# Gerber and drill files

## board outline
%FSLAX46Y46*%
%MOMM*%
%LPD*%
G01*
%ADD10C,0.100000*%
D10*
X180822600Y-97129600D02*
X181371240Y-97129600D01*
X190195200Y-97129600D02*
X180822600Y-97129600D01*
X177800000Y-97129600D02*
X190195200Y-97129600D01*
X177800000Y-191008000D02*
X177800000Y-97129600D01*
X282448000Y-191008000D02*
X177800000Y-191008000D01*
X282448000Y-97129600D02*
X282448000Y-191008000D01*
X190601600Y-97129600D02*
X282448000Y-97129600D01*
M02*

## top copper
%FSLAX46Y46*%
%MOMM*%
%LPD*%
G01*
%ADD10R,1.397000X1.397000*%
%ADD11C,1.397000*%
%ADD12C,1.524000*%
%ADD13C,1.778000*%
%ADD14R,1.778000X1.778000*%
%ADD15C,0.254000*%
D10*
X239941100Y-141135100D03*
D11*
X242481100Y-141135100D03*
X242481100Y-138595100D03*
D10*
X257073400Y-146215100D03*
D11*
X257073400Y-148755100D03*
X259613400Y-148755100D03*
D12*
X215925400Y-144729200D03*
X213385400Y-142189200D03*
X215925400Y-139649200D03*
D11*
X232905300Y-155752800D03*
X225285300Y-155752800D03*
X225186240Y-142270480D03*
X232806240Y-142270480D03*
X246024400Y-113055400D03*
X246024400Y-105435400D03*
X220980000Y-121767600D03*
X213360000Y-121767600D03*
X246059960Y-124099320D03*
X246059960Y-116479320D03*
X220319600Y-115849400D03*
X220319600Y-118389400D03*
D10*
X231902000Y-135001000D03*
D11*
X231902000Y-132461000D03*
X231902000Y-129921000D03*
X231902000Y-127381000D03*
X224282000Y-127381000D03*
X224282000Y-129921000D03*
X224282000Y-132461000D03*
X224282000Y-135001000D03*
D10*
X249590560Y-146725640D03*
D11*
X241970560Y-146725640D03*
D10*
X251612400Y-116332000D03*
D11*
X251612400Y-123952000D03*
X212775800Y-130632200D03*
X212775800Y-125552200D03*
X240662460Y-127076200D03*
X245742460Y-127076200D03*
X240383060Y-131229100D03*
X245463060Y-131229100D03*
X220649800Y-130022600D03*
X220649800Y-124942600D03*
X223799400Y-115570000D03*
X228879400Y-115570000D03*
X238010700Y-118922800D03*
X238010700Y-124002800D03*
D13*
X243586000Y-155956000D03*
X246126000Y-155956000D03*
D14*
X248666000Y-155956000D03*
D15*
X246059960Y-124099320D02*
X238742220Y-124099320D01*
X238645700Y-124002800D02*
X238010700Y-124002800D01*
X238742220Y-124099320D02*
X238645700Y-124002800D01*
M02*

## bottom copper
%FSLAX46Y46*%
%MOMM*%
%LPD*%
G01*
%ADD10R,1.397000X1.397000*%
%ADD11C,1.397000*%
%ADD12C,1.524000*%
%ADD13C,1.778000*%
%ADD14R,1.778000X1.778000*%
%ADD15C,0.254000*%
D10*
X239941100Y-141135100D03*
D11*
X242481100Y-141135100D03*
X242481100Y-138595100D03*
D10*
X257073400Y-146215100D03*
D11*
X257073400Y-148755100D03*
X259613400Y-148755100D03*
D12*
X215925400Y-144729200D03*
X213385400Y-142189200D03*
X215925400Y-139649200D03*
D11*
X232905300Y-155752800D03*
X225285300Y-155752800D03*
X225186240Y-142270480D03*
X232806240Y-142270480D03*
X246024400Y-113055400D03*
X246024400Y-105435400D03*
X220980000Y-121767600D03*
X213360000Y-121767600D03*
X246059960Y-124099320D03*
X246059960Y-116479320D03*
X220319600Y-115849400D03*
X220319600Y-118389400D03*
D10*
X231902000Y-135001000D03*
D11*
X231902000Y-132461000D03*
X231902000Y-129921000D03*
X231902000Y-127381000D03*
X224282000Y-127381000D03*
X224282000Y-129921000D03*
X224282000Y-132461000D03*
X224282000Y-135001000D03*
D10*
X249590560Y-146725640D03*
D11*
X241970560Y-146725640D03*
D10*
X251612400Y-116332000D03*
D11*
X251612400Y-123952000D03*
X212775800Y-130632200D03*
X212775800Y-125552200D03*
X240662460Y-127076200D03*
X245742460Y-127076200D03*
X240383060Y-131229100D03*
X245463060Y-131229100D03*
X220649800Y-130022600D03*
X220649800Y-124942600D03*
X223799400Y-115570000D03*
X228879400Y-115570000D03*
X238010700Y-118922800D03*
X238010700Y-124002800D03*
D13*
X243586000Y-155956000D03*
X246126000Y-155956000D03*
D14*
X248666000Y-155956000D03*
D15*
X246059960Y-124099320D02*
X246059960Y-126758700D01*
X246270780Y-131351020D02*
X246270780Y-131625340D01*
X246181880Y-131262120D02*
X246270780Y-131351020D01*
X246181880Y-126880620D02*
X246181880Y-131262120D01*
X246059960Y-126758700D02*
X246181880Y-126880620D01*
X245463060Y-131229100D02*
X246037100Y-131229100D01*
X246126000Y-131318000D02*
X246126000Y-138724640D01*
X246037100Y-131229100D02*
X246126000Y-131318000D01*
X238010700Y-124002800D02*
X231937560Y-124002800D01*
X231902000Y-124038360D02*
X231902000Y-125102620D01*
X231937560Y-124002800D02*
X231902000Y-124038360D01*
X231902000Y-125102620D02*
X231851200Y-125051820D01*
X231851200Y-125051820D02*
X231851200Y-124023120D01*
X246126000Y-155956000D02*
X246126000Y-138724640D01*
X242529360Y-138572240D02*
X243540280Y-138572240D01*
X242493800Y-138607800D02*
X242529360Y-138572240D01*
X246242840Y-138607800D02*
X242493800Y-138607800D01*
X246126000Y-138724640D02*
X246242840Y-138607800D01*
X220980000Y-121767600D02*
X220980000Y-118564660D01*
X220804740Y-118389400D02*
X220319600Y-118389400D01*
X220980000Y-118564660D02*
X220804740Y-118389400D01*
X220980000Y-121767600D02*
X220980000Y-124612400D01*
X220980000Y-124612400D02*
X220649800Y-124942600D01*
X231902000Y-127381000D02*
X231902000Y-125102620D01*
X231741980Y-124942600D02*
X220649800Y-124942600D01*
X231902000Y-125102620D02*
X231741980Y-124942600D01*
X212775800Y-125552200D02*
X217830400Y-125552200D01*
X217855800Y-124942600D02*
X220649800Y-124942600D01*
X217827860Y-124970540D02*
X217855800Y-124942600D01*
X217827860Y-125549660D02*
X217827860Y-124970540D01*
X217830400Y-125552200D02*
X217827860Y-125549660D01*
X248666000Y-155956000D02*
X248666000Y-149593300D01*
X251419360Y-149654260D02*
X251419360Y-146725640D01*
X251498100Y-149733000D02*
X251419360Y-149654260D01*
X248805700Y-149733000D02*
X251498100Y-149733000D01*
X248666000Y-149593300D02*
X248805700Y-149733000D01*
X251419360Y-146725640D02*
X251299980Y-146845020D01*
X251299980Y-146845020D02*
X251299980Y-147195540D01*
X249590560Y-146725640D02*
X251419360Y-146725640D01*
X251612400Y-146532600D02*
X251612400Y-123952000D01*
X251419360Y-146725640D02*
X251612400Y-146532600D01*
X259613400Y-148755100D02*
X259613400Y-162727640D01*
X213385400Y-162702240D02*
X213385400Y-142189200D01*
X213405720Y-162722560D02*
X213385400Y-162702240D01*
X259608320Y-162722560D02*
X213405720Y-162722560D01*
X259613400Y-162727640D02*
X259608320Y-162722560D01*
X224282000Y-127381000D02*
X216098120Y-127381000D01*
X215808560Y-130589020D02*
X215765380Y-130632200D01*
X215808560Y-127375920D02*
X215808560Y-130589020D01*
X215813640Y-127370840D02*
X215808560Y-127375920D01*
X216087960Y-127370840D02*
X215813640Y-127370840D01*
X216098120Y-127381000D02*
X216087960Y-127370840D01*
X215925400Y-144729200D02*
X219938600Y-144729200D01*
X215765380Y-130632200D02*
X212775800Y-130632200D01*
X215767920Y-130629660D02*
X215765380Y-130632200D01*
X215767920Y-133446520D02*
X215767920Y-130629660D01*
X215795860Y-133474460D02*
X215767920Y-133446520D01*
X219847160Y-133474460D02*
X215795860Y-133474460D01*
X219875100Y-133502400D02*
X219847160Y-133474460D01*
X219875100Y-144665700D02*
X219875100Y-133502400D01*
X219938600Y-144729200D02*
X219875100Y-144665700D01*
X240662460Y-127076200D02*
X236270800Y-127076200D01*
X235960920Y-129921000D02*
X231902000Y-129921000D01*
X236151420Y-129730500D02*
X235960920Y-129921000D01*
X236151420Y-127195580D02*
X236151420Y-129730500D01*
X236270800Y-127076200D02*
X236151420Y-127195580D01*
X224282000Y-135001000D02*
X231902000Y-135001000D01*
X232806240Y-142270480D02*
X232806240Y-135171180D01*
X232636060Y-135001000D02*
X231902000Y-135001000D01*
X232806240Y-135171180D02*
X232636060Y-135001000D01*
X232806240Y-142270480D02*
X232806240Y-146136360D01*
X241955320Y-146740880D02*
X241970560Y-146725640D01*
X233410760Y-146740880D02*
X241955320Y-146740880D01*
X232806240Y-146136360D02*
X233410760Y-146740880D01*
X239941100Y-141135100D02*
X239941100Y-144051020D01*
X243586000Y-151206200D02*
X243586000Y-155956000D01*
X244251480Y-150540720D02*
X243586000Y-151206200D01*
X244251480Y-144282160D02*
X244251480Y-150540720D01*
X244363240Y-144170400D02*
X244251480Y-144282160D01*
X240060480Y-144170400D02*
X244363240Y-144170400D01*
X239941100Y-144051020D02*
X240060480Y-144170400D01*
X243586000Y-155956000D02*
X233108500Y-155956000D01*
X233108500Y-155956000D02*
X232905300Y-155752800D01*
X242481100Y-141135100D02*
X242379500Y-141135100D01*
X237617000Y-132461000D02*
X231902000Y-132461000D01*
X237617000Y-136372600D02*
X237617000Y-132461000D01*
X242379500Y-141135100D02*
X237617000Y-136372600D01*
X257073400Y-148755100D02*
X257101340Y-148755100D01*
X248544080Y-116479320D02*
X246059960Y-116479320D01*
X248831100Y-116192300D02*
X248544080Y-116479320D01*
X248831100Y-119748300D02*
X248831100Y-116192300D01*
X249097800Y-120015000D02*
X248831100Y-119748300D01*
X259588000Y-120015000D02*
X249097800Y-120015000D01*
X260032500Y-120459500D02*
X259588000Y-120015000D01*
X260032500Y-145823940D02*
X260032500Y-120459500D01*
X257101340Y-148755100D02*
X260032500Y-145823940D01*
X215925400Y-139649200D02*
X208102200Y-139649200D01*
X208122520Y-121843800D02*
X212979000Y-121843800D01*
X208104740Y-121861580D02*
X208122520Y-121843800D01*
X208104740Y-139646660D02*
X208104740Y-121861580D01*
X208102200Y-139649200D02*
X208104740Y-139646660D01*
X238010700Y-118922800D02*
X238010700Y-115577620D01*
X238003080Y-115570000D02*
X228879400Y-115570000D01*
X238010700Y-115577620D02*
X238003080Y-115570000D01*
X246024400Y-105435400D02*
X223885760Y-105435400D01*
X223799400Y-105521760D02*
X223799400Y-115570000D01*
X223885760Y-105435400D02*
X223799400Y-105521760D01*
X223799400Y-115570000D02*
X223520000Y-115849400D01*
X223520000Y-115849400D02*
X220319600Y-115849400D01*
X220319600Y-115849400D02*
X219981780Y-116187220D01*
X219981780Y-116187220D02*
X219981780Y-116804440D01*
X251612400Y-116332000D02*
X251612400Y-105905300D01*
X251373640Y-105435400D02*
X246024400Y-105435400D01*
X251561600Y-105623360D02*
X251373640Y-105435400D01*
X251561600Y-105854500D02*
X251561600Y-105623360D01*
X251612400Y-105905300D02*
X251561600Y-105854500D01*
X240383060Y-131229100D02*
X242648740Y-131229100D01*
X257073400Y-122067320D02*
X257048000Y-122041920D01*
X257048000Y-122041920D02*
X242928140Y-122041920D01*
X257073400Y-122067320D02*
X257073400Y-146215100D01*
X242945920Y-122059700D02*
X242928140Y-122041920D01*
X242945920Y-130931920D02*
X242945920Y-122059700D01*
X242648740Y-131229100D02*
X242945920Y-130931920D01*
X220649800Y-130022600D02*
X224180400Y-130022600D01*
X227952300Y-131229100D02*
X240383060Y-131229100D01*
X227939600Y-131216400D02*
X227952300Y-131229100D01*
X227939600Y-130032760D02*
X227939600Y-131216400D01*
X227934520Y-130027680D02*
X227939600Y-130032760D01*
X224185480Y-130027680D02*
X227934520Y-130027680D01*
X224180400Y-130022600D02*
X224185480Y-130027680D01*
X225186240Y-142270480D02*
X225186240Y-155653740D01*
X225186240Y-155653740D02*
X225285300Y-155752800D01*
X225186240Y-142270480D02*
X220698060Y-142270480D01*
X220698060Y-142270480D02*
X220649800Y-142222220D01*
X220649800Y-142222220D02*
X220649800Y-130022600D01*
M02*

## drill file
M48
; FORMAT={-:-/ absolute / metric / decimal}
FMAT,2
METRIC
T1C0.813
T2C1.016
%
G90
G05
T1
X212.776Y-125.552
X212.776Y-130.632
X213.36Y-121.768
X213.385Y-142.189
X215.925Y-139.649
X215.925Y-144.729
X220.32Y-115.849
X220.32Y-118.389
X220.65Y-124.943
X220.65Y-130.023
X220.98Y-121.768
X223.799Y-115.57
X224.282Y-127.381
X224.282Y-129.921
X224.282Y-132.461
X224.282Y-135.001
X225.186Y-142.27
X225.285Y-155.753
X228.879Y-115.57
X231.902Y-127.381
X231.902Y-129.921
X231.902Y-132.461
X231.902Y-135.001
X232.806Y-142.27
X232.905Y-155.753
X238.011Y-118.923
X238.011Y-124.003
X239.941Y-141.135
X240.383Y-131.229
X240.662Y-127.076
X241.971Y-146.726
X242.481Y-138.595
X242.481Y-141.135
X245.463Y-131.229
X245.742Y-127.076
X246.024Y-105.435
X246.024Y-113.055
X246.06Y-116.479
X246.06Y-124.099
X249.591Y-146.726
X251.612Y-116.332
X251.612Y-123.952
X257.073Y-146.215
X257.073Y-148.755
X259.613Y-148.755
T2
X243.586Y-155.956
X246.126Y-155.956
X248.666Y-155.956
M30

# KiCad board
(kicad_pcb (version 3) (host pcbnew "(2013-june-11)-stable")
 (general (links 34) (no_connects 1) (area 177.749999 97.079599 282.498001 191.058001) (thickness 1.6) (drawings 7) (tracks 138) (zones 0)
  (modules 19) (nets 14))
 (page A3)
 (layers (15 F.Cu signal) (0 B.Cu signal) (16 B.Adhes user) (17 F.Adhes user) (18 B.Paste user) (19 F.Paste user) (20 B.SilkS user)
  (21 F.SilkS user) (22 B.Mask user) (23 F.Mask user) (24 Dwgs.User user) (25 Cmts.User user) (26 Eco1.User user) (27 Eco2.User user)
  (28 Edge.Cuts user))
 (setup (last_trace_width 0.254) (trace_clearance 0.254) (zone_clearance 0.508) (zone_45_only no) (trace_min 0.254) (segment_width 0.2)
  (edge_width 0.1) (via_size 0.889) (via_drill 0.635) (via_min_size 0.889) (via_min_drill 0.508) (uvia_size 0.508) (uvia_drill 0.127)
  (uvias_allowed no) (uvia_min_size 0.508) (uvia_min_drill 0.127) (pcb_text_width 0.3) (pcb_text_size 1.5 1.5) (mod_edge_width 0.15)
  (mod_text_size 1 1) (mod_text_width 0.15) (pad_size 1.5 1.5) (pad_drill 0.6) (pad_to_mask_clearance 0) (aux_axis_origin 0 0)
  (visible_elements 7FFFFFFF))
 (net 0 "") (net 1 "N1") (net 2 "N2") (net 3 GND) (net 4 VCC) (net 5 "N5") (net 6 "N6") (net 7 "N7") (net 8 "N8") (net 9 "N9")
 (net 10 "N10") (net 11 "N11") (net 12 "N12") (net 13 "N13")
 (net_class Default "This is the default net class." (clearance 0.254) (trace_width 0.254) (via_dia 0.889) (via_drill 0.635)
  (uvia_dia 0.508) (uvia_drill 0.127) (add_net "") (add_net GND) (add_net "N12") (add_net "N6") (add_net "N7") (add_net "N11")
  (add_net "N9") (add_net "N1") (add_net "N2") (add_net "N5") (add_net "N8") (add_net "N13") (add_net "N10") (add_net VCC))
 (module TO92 (layer F.Cu) (at 241.2111 139.8651 180)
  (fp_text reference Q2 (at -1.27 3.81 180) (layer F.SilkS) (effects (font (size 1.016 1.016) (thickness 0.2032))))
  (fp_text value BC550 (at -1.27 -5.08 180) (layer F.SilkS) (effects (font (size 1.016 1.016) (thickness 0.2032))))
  (pad 1 thru_hole rect (at 1.27 -1.27 180) (size 1.397 1.397) (drill 0.8128) (layers *.Cu *.Mask F.SilkS) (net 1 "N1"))
  (pad 2 thru_hole circle (at -1.27 -1.27 180) (size 1.397 1.397) (drill 0.8128) (layers *.Cu *.Mask F.SilkS) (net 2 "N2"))
  (pad 3 thru_hole circle (at -1.27 1.27 180) (size 1.397 1.397) (drill 0.8128) (layers *.Cu *.Mask F.SilkS) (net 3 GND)))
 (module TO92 (layer F.Cu) (at 258.3434 147.4851 90)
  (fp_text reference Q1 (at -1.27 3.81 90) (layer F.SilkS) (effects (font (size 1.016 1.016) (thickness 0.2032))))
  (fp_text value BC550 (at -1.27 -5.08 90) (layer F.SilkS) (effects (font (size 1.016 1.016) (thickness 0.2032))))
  (pad 1 thru_hole rect (at 1.27 -1.27 90) (size 1.397 1.397) (drill 0.8128) (layers *.Cu *.Mask F.SilkS) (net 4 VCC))
  (pad 2 thru_hole circle (at -1.27 -1.27 90) (size 1.397 1.397) (drill 0.8128) (layers *.Cu *.Mask F.SilkS) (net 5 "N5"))
  (pad 3 thru_hole circle (at -1.27 1.27 90) (size 1.397 1.397) (drill 0.8128) (layers *.Cu *.Mask F.SilkS) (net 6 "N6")))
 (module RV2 (layer F.Cu) (at 214.6554 142.1892 90) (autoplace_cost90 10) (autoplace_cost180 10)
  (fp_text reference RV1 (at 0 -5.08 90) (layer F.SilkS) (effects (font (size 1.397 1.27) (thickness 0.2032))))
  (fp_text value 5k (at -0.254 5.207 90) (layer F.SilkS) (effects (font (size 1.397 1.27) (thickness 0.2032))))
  (pad 1 thru_hole circle (at -2.54 1.27 90) (size 1.524 1.524) (drill 0.8128) (layers *.Cu *.Mask F.SilkS) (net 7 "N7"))
  (pad 2 thru_hole circle (at 0 -1.27 90) (size 1.524 1.524) (drill 0.8128) (layers *.Cu *.Mask F.SilkS) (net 6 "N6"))
  (pad 3 thru_hole circle (at 2.54 1.27 90) (size 1.524 1.524) (drill 0.8128) (layers *.Cu *.Mask F.SilkS) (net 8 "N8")))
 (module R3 (layer F.Cu) (at 229.0953 155.7528 180) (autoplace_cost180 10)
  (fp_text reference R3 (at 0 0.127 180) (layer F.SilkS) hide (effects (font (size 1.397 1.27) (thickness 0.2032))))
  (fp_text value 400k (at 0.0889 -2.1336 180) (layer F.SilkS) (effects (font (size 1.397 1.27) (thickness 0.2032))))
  (pad 1 thru_hole circle (at -3.81 0 180) (size 1.397 1.397) (drill 0.8128) (layers *.Cu *.Mask F.SilkS) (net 1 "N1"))
  (pad 2 thru_hole circle (at 3.81 0 180) (size 1.397 1.397) (drill 0.8128) (layers *.Cu *.Mask F.SilkS) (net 4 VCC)))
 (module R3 (layer F.Cu) (at 228.99624 142.27048) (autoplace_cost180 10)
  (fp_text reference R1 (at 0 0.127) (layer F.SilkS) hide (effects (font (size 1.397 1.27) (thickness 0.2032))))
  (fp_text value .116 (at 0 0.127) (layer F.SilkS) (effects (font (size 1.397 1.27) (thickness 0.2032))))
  (pad 1 thru_hole circle (at -3.81 0) (size 1.397 1.397) (drill 0.8128) (layers *.Cu *.Mask F.SilkS) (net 4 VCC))
  (pad 2 thru_hole circle (at 3.81 0) (size 1.397 1.397) (drill 0.8128) (layers *.Cu *.Mask F.SilkS) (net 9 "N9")))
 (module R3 (layer F.Cu) (at 246.0244 109.2454 90) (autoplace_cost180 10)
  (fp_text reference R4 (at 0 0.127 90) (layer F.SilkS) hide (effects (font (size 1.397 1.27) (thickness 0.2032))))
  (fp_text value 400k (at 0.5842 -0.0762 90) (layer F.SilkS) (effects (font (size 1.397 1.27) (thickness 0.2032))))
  (pad 1 thru_hole circle (at -3.81 0 90) (size 1.397 1.397) (drill 0.8128) (layers *.Cu *.Mask F.SilkS) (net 5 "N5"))
  (pad 2 thru_hole circle (at 3.81 0 90) (size 1.397 1.397) (drill 0.8128) (layers *.Cu *.Mask F.SilkS) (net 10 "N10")))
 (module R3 (layer F.Cu) (at 217.17 121.7676 180) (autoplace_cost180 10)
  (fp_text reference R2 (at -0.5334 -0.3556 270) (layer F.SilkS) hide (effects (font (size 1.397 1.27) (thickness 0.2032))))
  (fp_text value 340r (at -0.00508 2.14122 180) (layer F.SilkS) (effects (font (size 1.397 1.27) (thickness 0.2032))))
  (pad 1 thru_hole circle (at -3.81 0 180) (size 1.397 1.397) (drill 0.8128) (layers *.Cu *.Mask F.SilkS) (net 3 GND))
  (pad 2 thru_hole circle (at 3.81 0 180) (size 1.397 1.397) (drill 0.8128) (layers *.Cu *.Mask F.SilkS) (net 8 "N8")))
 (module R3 (layer F.Cu) (at 246.05996 120.28932 90) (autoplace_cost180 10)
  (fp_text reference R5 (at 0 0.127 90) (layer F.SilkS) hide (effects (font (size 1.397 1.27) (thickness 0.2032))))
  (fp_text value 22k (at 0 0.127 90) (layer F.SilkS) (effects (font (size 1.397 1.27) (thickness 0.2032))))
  (pad 1 thru_hole circle (at -3.81 0 90) (size 1.397 1.397) (drill 0.8128) (layers *.Cu *.Mask F.SilkS) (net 3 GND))
  (pad 2 thru_hole circle (at 3.81 0 90) (size 1.397 1.397) (drill 0.8128) (layers *.Cu *.Mask F.SilkS) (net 5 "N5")))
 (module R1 (layer F.Cu) (at 220.3196 117.1194 270) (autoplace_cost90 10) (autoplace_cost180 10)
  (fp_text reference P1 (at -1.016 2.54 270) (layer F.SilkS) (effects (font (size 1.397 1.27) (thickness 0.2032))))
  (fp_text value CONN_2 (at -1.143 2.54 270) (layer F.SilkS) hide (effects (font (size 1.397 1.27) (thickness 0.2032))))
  (pad 1 thru_hole circle (at -1.27 0 270) (size 1.397 1.397) (drill 0.8128) (layers *.Cu *.Mask F.SilkS) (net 10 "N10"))
  (pad 2 thru_hole circle (at 1.27 0 270) (size 1.397 1.397) (drill 0.8128) (layers *.Cu *.Mask F.SilkS) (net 3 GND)))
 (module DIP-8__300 (layer F.Cu) (at 228.092 131.191 90)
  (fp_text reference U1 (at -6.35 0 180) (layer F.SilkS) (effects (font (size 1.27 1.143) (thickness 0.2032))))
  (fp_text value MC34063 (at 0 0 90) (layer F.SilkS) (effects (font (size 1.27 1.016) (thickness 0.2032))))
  (pad 1 thru_hole rect (at -3.81 3.81 90) (size 1.397 1.397) (drill 0.8128) (layers *.Cu *.Mask F.SilkS) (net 9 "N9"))
  (pad 2 thru_hole circle (at -1.27 3.81 90) (size 1.397 1.397) (drill 0.8128) (layers *.Cu *.Mask F.SilkS) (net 2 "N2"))
  (pad 3 thru_hole circle (at 1.27 3.81 90) (size 1.397 1.397) (drill 0.8128) (layers *.Cu *.Mask F.SilkS) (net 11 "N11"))
  (pad 4 thru_hole circle (at 3.81 3.81 90) (size 1.397 1.397) (drill 0.8128) (layers *.Cu *.Mask F.SilkS) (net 3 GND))
  (pad 5 thru_hole circle (at 3.81 -3.81 90) (size 1.397 1.397) (drill 0.8128) (layers *.Cu *.Mask F.SilkS) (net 7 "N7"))
  (pad 6 thru_hole circle (at 1.27 -3.81 90) (size 1.397 1.397) (drill 0.8128) (layers *.Cu *.Mask F.SilkS) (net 4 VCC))
  (pad 7 thru_hole circle (at -1.27 -3.81 90) (size 1.397 1.397) (drill 0.8128) (layers *.Cu *.Mask F.SilkS))
  (pad 8 thru_hole circle (at -3.81 -3.81 90) (size 1.397 1.397) (drill 0.8128) (layers *.Cu *.Mask F.SilkS) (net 9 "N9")))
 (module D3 (layer F.Cu) (at 245.78056 146.72564)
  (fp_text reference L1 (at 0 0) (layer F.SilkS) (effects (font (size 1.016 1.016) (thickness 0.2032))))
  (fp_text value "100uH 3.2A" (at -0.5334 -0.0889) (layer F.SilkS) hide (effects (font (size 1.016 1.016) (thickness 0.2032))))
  (pad 2 thru_hole rect (at 3.81 0) (size 1.397 1.397) (drill 0.8128) (layers *.Cu *.Mask F.SilkS) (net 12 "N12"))
  (pad 1 thru_hole circle (at -3.81 0) (size 1.397 1.397) (drill 0.8128) (layers *.Cu *.Mask F.SilkS) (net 9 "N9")))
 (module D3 (layer F.Cu) (at 251.6124 120.142 90)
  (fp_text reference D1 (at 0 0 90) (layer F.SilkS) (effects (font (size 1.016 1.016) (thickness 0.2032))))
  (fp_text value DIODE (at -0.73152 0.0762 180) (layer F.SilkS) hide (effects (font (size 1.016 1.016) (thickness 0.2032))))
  (pad 2 thru_hole rect (at 3.81 0 90) (size 1.397 1.397) (drill 0.8128) (layers *.Cu *.Mask F.SilkS) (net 10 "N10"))
  (pad 1 thru_hole circle (at -3.81 0 90) (size 1.397 1.397) (drill 0.8128) (layers *.Cu *.Mask F.SilkS) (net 12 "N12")))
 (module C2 (layer F.Cu) (at 212.7758 128.0922 90)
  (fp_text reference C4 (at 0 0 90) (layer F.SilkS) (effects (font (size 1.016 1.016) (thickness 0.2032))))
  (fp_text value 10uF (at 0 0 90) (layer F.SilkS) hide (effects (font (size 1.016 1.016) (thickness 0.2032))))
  (pad 1 thru_hole circle (at -2.54 0 90) (size 1.397 1.397) (drill 0.8128) (layers *.Cu *.Mask F.SilkS) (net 7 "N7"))
  (pad 2 thru_hole circle (at 2.54 0 90) (size 1.397 1.397) (drill 0.8128) (layers *.Cu *.Mask F.SilkS) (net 3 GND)))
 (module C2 (layer F.Cu) (at 243.20246 127.0762)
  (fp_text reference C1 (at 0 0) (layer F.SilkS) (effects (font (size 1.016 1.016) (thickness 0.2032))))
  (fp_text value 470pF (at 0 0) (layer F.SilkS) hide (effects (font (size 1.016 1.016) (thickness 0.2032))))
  (pad 1 thru_hole circle (at -2.54 0) (size 1.397 1.397) (drill 0.8128) (layers *.Cu *.Mask F.SilkS) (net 11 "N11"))
  (pad 2 thru_hole circle (at 2.54 0) (size 1.397 1.397) (drill 0.8128) (layers *.Cu *.Mask F.SilkS) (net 3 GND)))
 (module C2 (layer F.Cu) (at 242.92306 131.2291)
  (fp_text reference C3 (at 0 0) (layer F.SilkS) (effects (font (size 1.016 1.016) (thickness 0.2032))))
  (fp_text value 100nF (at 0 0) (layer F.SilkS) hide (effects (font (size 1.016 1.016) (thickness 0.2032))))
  (pad 1 thru_hole circle (at -2.54 0) (size 1.397 1.397) (drill 0.8128) (layers *.Cu *.Mask F.SilkS) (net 4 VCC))
  (pad 2 thru_hole circle (at 2.54 0) (size 1.397 1.397) (drill 0.8128) (layers *.Cu *.Mask F.SilkS) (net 3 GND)))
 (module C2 (layer F.Cu) (at 220.6498 127.4826 90)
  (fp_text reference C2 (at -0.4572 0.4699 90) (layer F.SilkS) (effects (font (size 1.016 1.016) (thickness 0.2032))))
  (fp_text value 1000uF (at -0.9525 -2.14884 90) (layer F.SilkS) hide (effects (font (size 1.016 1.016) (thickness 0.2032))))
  (pad 1 thru_hole circle (at -2.54 0 90) (size 1.397 1.397) (drill 0.8128) (layers *.Cu *.Mask F.SilkS) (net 4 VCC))
  (pad 2 thru_hole circle (at 2.54 0 90) (size 1.397 1.397) (drill 0.8128) (layers *.Cu *.Mask F.SilkS) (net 3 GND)))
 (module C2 (layer F.Cu) (at 226.3394 115.57)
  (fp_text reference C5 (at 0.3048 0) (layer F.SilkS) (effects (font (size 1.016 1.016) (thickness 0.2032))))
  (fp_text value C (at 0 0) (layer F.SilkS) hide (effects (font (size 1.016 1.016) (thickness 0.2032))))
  (pad 1 thru_hole circle (at -2.54 0) (size 1.397 1.397) (drill 0.8128) (layers *.Cu *.Mask F.SilkS) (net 10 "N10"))
  (pad 2 thru_hole circle (at 2.54 0) (size 1.397 1.397) (drill 0.8128) (layers *.Cu *.Mask F.SilkS) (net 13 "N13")))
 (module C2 (layer F.Cu) (at 238.0107 121.4628 270)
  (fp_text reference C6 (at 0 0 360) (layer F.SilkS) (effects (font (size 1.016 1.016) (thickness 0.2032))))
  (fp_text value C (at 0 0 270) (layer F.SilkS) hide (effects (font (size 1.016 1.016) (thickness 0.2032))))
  (pad 1 thru_hole circle (at -2.54 0 270) (size 1.397 1.397) (drill 0.8128) (layers *.Cu *.Mask F.SilkS) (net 13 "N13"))
  (pad 2 thru_hole circle (at 2.54 0 270) (size 1.397 1.397) (drill 0.8128) (layers *.Cu *.Mask F.SilkS) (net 3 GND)))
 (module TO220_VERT (layer F.Cu) (at 246.126 155.956 90)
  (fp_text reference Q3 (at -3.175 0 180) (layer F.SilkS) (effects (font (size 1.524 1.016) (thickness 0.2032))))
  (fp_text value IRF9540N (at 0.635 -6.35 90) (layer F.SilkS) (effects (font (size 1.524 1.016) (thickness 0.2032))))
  (pad 2 thru_hole circle (at 0 -2.54 90) (size 1.778 1.778) (drill 1.016) (layers *.Cu *.Mask F.SilkS) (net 1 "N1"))
  (pad 3 thru_hole circle (at 0 0 90) (size 1.778 1.778) (drill 1.016) (layers *.Cu *.Mask F.SilkS) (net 3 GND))
  (pad 1 thru_hole rect (at 0 2.54 90) (size 1.778 1.778) (drill 1.016) (layers *.Cu *.Mask F.SilkS) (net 12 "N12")))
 (gr_line (start 180.8226 97.1296) (end 181.37124 97.1296) (angle 90) (layer Edge.Cuts) (width 0.1))
 (gr_line (start 190.1952 97.1296) (end 180.8226 97.1296) (angle 90) (layer Edge.Cuts) (width 0.1))
 (gr_line (start 177.8 97.1296) (end 190.1952 97.1296) (angle 90) (layer Edge.Cuts) (width 0.1))
 (gr_line (start 177.8 191.008) (end 177.8 97.1296) (angle 90) (layer Edge.Cuts) (width 0.1))
 (gr_line (start 282.448 191.008) (end 177.8 191.008) (angle 90) (layer Edge.Cuts) (width 0.1))
 (gr_line (start 282.448 97.1296) (end 282.448 191.008) (angle 90) (layer Edge.Cuts) (width 0.1))
 (gr_line (start 190.6016 97.1296) (end 282.448 97.1296) (angle 90) (layer Edge.Cuts) (width 0.1))
 (segment (start 246.05996 124.09932) (end 246.05996 126.7587) (width 0.254) (layer B.Cu) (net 3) (status C00000))
 (segment (start 246.27078 131.35102) (end 246.27078 131.62534) (width 0.254) (layer B.Cu) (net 3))
 (segment (start 246.18188 131.26212) (end 246.27078 131.35102) (width 0.254) (layer B.Cu) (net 3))
 (segment (start 246.18188 126.88062) (end 246.18188 131.26212) (width 0.254) (layer B.Cu) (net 3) (status 400000))
 (segment (start 246.05996 126.7587) (end 246.18188 126.88062) (width 0.254) (layer B.Cu) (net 3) (status C00000))
 (segment (start 245.46306 131.2291) (end 246.0371 131.2291) (width 0.254) (layer B.Cu) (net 3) (status C00000))
 (segment (start 246.126 131.318) (end 246.126 138.72464) (width 0.254) (layer B.Cu) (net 3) (status 400000))
 (segment (start 246.0371 131.2291) (end 246.126 131.318) (width 0.254) (layer B.Cu) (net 3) (status C00000))
 (segment (start 238.0107 124.0028) (end 231.93756 124.0028) (width 0.254) (layer B.Cu) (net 3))
 (segment (start 231.902 124.03836) (end 231.902 125.10262) (width 0.254) (layer B.Cu) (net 3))
 (segment (start 231.93756 124.0028) (end 231.902 124.03836) (width 0.254) (layer B.Cu) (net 3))
 (segment (start 231.902 125.10262) (end 231.8512 125.05182) (width 0.254) (layer B.Cu) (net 3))
 (segment (start 231.8512 125.05182) (end 231.8512 124.02312) (width 0.254) (layer B.Cu) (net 3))
 (segment (start 246.05996 124.09932) (end 238.74222 124.09932) (width 0.254) (layer F.Cu) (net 3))
 (segment (start 238.6457 124.0028) (end 238.0107 124.0028) (width 0.254) (layer F.Cu) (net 3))
 (segment (start 238.74222 124.09932) (end 238.6457 124.0028) (width 0.254) (layer F.Cu) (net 3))
 (segment (start 246.126 155.956) (end 246.126 138.72464) (width 0.254) (layer B.Cu) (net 3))
 (segment (start 242.52936 138.57224) (end 243.54028 138.57224) (width 0.254) (layer B.Cu) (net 3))
 (segment (start 242.4938 138.6078) (end 242.52936 138.57224) (width 0.254) (layer B.Cu) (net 3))
 (segment (start 246.24284 138.6078) (end 242.4938 138.6078) (width 0.254) (layer B.Cu) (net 3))
 (segment (start 246.126 138.72464) (end 246.24284 138.6078) (width 0.254) (layer B.Cu) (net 3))
 (segment (start 220.98 121.7676) (end 220.98 118.56466) (width 0.254) (layer B.Cu) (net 3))
 (segment (start 220.80474 118.3894) (end 220.3196 118.3894) (width 0.254) (layer B.Cu) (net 3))
 (segment (start 220.98 118.56466) (end 220.80474 118.3894) (width 0.254) (layer B.Cu) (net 3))
 (segment (start 220.98 121.7676) (end 220.98 124.6124) (width 0.254) (layer B.Cu) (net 3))
 (segment (start 220.98 124.6124) (end 220.6498 124.9426) (width 0.254) (layer B.Cu) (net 3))
 (segment (start 231.902 127.381) (end 231.902 125.10262) (width 0.254) (layer B.Cu) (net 3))
 (segment (start 231.74198 124.9426) (end 220.6498 124.9426) (width 0.254) (layer B.Cu) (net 3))
 (segment (start 231.902 125.10262) (end 231.74198 124.9426) (width 0.254) (layer B.Cu) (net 3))
 (segment (start 212.7758 125.5522) (end 217.8304 125.5522) (width 0.254) (layer B.Cu) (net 3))
 (segment (start 217.8558 124.9426) (end 220.6498 124.9426) (width 0.254) (layer B.Cu) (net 3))
 (segment (start 217.82786 124.97054) (end 217.8558 124.9426) (width 0.254) (layer B.Cu) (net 3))
 (segment (start 217.82786 125.54966) (end 217.82786 124.97054) (width 0.254) (layer B.Cu) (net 3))
 (segment (start 217.8304 125.5522) (end 217.82786 125.54966) (width 0.254) (layer B.Cu) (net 3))
 (segment (start 248.666 155.956) (end 248.666 149.5933) (width 0.254) (layer B.Cu) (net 12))
 (segment (start 251.41936 149.65426) (end 251.41936 146.72564) (width 0.254) (layer B.Cu) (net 12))
 (segment (start 251.4981 149.733) (end 251.41936 149.65426) (width 0.254) (layer B.Cu) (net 12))
 (segment (start 248.8057 149.733) (end 251.4981 149.733) (width 0.254) (layer B.Cu) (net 12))
 (segment (start 248.666 149.5933) (end 248.8057 149.733) (width 0.254) (layer B.Cu) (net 12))
 (segment (start 251.41936 146.72564) (end 251.29998 146.84502) (width 0.254) (layer B.Cu) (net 12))
 (segment (start 251.29998 146.84502) (end 251.29998 147.19554) (width 0.254) (layer B.Cu) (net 12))
 (segment (start 249.59056 146.72564) (end 251.41936 146.72564) (width 0.254) (layer B.Cu) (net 12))
 (segment (start 251.6124 146.5326) (end 251.6124 123.952) (width 0.254) (layer B.Cu) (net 12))
 (segment (start 251.41936 146.72564) (end 251.6124 146.5326) (width 0.254) (layer B.Cu) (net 12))
 (segment (start 259.6134 148.7551) (end 259.6134 162.72764) (width 0.254) (layer B.Cu) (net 6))
 (segment (start 213.3854 162.70224) (end 213.3854 142.1892) (width 0.254) (layer B.Cu) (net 6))
 (segment (start 213.40572 162.72256) (end 213.3854 162.70224) (width 0.254) (layer B.Cu) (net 6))
 (segment (start 259.60832 162.72256) (end 213.40572 162.72256) (width 0.254) (layer B.Cu) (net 6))
 (segment (start 259.6134 162.72764) (end 259.60832 162.72256) (width 0.254) (layer B.Cu) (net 6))
 (segment (start 224.282 127.381) (end 216.09812 127.381) (width 0.254) (layer B.Cu) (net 7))
 (segment (start 215.80856 130.58902) (end 215.76538 130.6322) (width 0.254) (layer B.Cu) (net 7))
 (segment (start 215.80856 127.37592) (end 215.80856 130.58902) (width 0.254) (layer B.Cu) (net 7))
 (segment (start 215.81364 127.37084) (end 215.80856 127.37592) (width 0.254) (layer B.Cu) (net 7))
 (segment (start 216.08796 127.37084) (end 215.81364 127.37084) (width 0.254) (layer B.Cu) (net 7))
 (segment (start 216.09812 127.381) (end 216.08796 127.37084) (width 0.254) (layer B.Cu) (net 7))
 (segment (start 215.9254 144.7292) (end 219.9386 144.7292) (width 0.254) (layer B.Cu) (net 7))
 (segment (start 215.76538 130.6322) (end 212.7758 130.6322) (width 0.254) (layer B.Cu) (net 7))
 (segment (start 215.76792 130.62966) (end 215.76538 130.6322) (width 0.254) (layer B.Cu) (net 7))
 (segment (start 215.76792 133.44652) (end 215.76792 130.62966) (width 0.254) (layer B.Cu) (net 7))
 (segment (start 215.79586 133.47446) (end 215.76792 133.44652) (width 0.254) (layer B.Cu) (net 7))
 (segment (start 219.84716 133.47446) (end 215.79586 133.47446) (width 0.254) (layer B.Cu) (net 7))
 (segment (start 219.8751 133.5024) (end 219.84716 133.47446) (width 0.254) (layer B.Cu) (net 7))
 (segment (start 219.8751 144.6657) (end 219.8751 133.5024) (width 0.254) (layer B.Cu) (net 7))
 (segment (start 219.9386 144.7292) (end 219.8751 144.6657) (width 0.254) (layer B.Cu) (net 7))
 (segment (start 240.66246 127.0762) (end 236.2708 127.0762) (width 0.254) (layer B.Cu) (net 11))
 (segment (start 235.96092 129.921) (end 231.902 129.921) (width 0.254) (layer B.Cu) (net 11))
 (segment (start 236.15142 129.7305) (end 235.96092 129.921) (width 0.254) (layer B.Cu) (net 11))
 (segment (start 236.15142 127.19558) (end 236.15142 129.7305) (width 0.254) (layer B.Cu) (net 11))
 (segment (start 236.2708 127.0762) (end 236.15142 127.19558) (width 0.254) (layer B.Cu) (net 11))
 (segment (start 224.282 135.001) (end 231.902 135.001) (width 0.254) (layer B.Cu) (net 9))
 (segment (start 232.80624 142.27048) (end 232.80624 135.17118) (width 0.254) (layer B.Cu) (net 9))
 (segment (start 232.63606 135.001) (end 231.902 135.001) (width 0.254) (layer B.Cu) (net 9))
 (segment (start 232.80624 135.17118) (end 232.63606 135.001) (width 0.254) (layer B.Cu) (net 9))
 (segment (start 232.80624 142.27048) (end 232.80624 146.13636) (width 0.254) (layer B.Cu) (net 9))
 (segment (start 241.95532 146.74088) (end 241.97056 146.72564) (width 0.254) (layer B.Cu) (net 9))
 (segment (start 233.41076 146.74088) (end 241.95532 146.74088) (width 0.254) (layer B.Cu) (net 9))
 (segment (start 232.80624 146.13636) (end 233.41076 146.74088) (width 0.254) (layer B.Cu) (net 9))
 (segment (start 239.9411 141.1351) (end 239.9411 144.05102) (width 0.254) (layer B.Cu) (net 1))
 (segment (start 243.586 151.2062) (end 243.586 155.956) (width 0.254) (layer B.Cu) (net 1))
 (segment (start 244.25148 150.54072) (end 243.586 151.2062) (width 0.254) (layer B.Cu) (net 1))
 (segment (start 244.25148 144.28216) (end 244.25148 150.54072) (width 0.254) (layer B.Cu) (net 1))
 (segment (start 244.36324 144.1704) (end 244.25148 144.28216) (width 0.254) (layer B.Cu) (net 1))
 (segment (start 240.06048 144.1704) (end 244.36324 144.1704) (width 0.254) (layer B.Cu) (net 1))
 (segment (start 239.9411 144.05102) (end 240.06048 144.1704) (width 0.254) (layer B.Cu) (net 1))
 (segment (start 243.586 155.956) (end 233.1085 155.956) (width 0.254) (layer B.Cu) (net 1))
 (segment (start 233.1085 155.956) (end 232.9053 155.7528) (width 0.254) (layer B.Cu) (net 1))
 (segment (start 242.4811 141.1351) (end 242.3795 141.1351) (width 0.254) (layer B.Cu) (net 2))
 (segment (start 237.617 132.461) (end 231.902 132.461) (width 0.254) (layer B.Cu) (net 2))
 (segment (start 237.617 136.3726) (end 237.617 132.461) (width 0.254) (layer B.Cu) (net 2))
 (segment (start 242.3795 141.1351) (end 237.617 136.3726) (width 0.254) (layer B.Cu) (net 2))
 (segment (start 257.0734 148.7551) (end 257.10134 148.7551) (width 0.254) (layer B.Cu) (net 5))
 (segment (start 248.54408 116.47932) (end 246.05996 116.47932) (width 0.254) (layer B.Cu) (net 5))
 (segment (start 248.8311 116.1923) (end 248.54408 116.47932) (width 0.254) (layer B.Cu) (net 5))
 (segment (start 248.8311 119.7483) (end 248.8311 116.1923) (width 0.254) (layer B.Cu) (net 5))
 (segment (start 249.0978 120.015) (end 248.8311 119.7483) (width 0.254) (layer B.Cu) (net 5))
 (segment (start 259.588 120.015) (end 249.0978 120.015) (width 0.254) (layer B.Cu) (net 5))
 (segment (start 260.0325 120.4595) (end 259.588 120.015) (width 0.254) (layer B.Cu) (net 5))
 (segment (start 260.0325 145.82394) (end 260.0325 120.4595) (width 0.254) (layer B.Cu) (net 5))
 (segment (start 257.10134 148.7551) (end 260.0325 145.82394) (width 0.254) (layer B.Cu) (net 5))
 (segment (start 215.9254 139.6492) (end 208.1022 139.6492) (width 0.254) (layer B.Cu) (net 8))
 (segment (start 208.12252 121.8438) (end 212.979 121.8438) (width 0.254) (layer B.Cu) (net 8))
 (segment (start 208.10474 121.86158) (end 208.12252 121.8438) (width 0.254) (layer B.Cu) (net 8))
 (segment (start 208.10474 139.64666) (end 208.10474 121.86158) (width 0.254) (layer B.Cu) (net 8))
 (segment (start 208.1022 139.6492) (end 208.10474 139.64666) (width 0.254) (layer B.Cu) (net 8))
 (segment (start 238.0107 118.9228) (end 238.0107 115.57762) (width 0.254) (layer B.Cu) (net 13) (status 400000))
 (segment (start 238.00308 115.57) (end 228.8794 115.57) (width 0.254) (layer B.Cu) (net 13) (status 800000))
 (segment (start 238.0107 115.57762) (end 238.00308 115.57) (width 0.254) (layer B.Cu) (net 13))
 (segment (start 246.0244 105.4354) (end 223.88576 105.4354) (width 0.254) (layer B.Cu) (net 10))
 (segment (start 223.7994 105.52176) (end 223.7994 115.57) (width 0.254) (layer B.Cu) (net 10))
 (segment (start 223.88576 105.4354) (end 223.7994 105.52176) (width 0.254) (layer B.Cu) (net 10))
 (segment (start 223.7994 115.57) (end 223.52 115.8494) (width 0.254) (layer B.Cu) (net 10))
 (segment (start 223.52 115.8494) (end 220.3196 115.8494) (width 0.254) (layer B.Cu) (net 10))
 (segment (start 220.3196 115.8494) (end 219.98178 116.18722) (width 0.254) (layer B.Cu) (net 10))
 (segment (start 219.98178 116.18722) (end 219.98178 116.80444) (width 0.254) (layer B.Cu) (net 10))
 (segment (start 251.6124 116.332) (end 251.6124 105.9053) (width 0.254) (layer B.Cu) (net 10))
 (segment (start 251.37364 105.4354) (end 246.0244 105.4354) (width 0.254) (layer B.Cu) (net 10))
 (segment (start 251.5616 105.62336) (end 251.37364 105.4354) (width 0.254) (layer B.Cu) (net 10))
 (segment (start 251.5616 105.8545) (end 251.5616 105.62336) (width 0.254) (layer B.Cu) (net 10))
 (segment (start 251.6124 105.9053) (end 251.5616 105.8545) (width 0.254) (layer B.Cu) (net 10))
 (segment (start 240.38306 131.2291) (end 242.64874 131.2291) (width 0.254) (layer B.Cu) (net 4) (status 400000))
 (segment (start 257.0734 122.06732) (end 257.048 122.04192) (width 0.254) (layer B.Cu) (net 4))
 (segment (start 257.048 122.04192) (end 242.92814 122.04192) (width 0.254) (layer B.Cu) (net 4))
 (segment (start 257.0734 122.06732) (end 257.0734 146.2151) (width 0.254) (layer B.Cu) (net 4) (status 800000))
 (segment (start 242.94592 122.0597) (end 242.92814 122.04192) (width 0.254) (layer B.Cu) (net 4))
 (segment (start 242.94592 130.93192) (end 242.94592 122.0597) (width 0.254) (layer B.Cu) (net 4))
 (segment (start 242.64874 131.2291) (end 242.94592 130.93192) (width 0.254) (layer B.Cu) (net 4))
 (segment (start 220.6498 130.0226) (end 224.1804 130.0226) (width 0.254) (layer B.Cu) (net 4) (status C00000))
 (segment (start 227.9523 131.2291) (end 240.38306 131.2291) (width 0.254) (layer B.Cu) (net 4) (status 800000))
 (segment (start 227.9396 131.2164) (end 227.9523 131.2291) (width 0.254) (layer B.Cu) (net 4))
 (segment (start 227.9396 130.03276) (end 227.9396 131.2164) (width 0.254) (layer B.Cu) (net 4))
 (segment (start 227.93452 130.02768) (end 227.9396 130.03276) (width 0.254) (layer B.Cu) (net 4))
 (segment (start 224.18548 130.02768) (end 227.93452 130.02768) (width 0.254) (layer B.Cu) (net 4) (status 400000))
 (segment (start 224.1804 130.0226) (end 224.18548 130.02768) (width 0.254) (layer B.Cu) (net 4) (status C00000))
 (segment (start 225.18624 142.27048) (end 225.18624 155.65374) (width 0.254) (layer B.Cu) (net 4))
 (segment (start 225.18624 155.65374) (end 225.2853 155.7528) (width 0.254) (layer B.Cu) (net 4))
 (segment (start 225.18624 142.27048) (end 220.69806 142.27048) (width 0.254) (layer B.Cu) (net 4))
 (segment (start 220.69806 142.27048) (end 220.6498 142.22222) (width 0.254) (layer B.Cu) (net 4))
 (segment (start 220.6498 142.22222) (end 220.6498 130.0226) (width 0.254) (layer B.Cu) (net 4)))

